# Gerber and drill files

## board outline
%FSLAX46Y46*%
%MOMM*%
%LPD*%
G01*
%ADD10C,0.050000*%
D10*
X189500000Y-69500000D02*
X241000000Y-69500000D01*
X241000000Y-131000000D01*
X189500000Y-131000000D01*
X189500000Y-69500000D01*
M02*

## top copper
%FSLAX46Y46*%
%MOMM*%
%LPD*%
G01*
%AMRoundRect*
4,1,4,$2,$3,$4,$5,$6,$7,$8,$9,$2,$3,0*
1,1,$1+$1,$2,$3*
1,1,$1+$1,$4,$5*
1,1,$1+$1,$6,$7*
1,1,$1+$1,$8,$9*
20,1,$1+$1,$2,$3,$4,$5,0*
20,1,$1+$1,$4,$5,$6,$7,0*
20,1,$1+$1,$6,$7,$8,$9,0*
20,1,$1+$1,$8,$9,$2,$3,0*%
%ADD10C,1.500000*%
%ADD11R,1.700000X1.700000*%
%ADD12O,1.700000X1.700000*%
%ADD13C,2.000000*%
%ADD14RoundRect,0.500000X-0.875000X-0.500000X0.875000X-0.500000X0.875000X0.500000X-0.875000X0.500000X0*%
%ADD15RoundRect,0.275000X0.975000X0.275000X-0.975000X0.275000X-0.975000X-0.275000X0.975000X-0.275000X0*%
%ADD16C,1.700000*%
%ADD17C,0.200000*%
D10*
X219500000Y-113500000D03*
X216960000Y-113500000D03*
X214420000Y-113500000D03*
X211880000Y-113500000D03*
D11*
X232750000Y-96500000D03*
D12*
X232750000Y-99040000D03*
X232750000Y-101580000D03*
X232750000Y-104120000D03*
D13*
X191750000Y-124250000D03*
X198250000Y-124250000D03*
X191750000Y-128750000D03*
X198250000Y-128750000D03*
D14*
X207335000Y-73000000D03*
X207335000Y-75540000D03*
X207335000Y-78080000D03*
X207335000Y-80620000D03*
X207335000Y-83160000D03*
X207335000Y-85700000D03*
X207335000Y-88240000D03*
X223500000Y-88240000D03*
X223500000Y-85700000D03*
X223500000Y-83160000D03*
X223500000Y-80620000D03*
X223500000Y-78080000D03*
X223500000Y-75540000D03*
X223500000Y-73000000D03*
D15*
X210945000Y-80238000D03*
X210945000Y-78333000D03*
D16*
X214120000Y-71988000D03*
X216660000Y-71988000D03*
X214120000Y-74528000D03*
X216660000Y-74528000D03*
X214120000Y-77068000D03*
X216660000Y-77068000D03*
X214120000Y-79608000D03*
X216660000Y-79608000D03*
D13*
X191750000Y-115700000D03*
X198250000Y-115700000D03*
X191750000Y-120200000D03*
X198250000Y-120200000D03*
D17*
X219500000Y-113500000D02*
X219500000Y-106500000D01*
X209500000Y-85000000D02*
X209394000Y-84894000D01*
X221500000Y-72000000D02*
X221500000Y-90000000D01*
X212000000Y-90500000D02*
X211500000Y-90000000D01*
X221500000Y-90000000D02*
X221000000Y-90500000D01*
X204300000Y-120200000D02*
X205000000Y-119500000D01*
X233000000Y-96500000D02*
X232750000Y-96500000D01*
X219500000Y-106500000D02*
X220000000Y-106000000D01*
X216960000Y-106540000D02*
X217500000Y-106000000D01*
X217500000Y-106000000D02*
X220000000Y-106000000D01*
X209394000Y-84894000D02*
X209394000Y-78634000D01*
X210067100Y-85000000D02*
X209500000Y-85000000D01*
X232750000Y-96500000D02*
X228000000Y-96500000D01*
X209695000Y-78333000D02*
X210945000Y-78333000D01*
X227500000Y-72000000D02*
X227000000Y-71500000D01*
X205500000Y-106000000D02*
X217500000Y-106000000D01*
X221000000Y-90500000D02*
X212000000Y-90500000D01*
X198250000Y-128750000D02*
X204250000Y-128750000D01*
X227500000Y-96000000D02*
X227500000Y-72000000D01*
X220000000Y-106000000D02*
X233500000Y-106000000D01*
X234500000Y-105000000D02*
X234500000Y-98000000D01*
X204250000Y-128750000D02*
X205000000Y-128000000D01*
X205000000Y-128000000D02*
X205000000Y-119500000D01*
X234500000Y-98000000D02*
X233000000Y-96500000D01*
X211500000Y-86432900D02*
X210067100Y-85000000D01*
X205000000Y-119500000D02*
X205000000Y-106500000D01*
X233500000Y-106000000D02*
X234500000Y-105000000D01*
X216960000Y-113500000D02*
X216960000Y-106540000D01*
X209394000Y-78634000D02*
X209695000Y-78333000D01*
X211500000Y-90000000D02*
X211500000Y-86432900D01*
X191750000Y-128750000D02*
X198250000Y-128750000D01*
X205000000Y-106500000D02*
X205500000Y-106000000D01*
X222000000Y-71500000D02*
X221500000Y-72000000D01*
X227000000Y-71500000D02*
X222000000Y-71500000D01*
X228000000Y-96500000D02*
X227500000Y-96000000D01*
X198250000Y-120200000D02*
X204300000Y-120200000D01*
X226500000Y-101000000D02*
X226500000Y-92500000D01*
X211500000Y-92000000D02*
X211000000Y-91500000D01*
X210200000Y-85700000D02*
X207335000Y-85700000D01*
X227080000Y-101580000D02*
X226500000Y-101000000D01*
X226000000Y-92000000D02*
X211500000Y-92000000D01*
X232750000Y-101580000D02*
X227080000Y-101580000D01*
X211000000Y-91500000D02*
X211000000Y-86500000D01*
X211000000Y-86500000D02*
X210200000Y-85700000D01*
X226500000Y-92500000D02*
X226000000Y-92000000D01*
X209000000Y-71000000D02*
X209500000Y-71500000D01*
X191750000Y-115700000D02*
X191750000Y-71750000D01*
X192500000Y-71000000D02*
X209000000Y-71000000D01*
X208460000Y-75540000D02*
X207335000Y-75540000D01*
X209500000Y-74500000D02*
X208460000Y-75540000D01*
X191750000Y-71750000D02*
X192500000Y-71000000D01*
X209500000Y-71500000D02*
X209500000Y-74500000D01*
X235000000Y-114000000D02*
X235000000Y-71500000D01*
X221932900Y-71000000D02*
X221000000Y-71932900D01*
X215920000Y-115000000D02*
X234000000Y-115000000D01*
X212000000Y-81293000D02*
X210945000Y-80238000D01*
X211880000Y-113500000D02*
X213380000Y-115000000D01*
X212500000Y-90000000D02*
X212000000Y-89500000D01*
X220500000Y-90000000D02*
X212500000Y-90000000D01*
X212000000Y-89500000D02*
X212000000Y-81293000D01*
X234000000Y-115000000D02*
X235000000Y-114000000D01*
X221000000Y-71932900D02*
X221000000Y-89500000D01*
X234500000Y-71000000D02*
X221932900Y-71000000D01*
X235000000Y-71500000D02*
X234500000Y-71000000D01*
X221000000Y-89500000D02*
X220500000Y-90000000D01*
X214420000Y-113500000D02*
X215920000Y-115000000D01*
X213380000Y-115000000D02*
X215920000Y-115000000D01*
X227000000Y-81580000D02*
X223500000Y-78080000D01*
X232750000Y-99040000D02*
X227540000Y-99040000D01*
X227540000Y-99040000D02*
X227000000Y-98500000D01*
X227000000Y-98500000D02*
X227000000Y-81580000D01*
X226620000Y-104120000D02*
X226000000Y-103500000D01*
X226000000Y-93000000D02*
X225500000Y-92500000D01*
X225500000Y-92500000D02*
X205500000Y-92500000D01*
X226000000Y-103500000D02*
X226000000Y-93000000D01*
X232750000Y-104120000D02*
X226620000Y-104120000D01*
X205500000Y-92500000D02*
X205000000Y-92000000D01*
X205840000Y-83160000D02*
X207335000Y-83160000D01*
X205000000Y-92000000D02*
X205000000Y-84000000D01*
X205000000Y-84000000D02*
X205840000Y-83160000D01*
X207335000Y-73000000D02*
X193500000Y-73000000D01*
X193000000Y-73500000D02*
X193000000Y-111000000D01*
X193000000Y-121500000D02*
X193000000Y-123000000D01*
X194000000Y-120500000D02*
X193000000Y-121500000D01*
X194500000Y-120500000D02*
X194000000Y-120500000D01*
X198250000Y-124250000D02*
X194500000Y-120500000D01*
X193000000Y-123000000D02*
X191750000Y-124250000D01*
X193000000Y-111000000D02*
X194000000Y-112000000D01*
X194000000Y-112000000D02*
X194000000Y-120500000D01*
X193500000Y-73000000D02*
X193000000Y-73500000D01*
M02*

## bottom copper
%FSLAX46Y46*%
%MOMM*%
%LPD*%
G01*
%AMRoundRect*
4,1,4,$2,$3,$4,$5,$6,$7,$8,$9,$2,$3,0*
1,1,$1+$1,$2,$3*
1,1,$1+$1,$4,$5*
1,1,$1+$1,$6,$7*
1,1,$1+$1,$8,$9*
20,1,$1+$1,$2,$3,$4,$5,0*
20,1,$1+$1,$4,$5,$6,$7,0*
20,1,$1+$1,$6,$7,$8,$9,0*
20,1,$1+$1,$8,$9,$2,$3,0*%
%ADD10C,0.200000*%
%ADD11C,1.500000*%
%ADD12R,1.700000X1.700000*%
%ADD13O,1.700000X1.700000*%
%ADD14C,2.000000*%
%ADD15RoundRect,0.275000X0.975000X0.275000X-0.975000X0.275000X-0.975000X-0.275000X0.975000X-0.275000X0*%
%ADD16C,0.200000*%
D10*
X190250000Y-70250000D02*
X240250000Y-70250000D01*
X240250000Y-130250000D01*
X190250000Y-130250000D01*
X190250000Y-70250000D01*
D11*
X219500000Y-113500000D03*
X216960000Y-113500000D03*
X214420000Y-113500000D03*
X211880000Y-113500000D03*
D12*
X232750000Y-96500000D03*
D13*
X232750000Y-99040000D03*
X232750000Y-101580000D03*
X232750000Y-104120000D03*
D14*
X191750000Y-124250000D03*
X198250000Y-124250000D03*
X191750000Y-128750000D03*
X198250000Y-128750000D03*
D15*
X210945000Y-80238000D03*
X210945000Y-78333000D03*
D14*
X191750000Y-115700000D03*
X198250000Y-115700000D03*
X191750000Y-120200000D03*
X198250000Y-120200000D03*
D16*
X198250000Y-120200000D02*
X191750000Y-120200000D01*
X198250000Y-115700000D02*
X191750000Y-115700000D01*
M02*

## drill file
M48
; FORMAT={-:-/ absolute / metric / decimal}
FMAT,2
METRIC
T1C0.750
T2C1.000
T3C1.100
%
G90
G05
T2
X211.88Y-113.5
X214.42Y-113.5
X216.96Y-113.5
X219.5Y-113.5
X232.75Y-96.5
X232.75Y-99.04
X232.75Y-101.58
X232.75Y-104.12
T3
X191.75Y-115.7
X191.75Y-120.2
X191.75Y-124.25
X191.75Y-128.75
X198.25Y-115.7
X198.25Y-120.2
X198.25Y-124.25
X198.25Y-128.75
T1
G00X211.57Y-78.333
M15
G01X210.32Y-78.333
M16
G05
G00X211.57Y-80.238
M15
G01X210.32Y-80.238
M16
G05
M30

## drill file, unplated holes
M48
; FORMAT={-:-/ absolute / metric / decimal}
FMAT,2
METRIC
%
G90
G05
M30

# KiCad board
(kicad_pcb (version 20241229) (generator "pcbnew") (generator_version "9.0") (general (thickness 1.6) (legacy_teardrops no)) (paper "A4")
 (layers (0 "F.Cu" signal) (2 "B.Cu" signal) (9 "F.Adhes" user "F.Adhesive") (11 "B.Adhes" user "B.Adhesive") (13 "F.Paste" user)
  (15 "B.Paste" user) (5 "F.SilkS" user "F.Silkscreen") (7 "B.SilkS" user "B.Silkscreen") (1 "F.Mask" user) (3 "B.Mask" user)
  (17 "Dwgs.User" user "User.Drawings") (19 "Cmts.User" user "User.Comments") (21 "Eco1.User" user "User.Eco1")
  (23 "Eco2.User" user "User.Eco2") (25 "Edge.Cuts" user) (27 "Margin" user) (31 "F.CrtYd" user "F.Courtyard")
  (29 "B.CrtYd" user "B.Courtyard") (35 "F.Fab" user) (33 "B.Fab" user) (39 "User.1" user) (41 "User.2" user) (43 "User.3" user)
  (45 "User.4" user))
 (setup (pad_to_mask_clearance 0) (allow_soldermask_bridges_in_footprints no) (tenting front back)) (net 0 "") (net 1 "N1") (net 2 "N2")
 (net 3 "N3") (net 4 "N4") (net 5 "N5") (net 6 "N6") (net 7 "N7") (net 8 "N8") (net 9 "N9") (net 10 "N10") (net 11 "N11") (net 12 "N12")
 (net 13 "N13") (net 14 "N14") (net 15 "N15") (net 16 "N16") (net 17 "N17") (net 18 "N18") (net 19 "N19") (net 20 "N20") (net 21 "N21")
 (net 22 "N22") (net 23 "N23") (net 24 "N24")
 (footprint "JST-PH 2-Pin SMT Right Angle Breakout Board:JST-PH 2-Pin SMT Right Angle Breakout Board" (layer "F.Cu") (at 206.66 119.59 90)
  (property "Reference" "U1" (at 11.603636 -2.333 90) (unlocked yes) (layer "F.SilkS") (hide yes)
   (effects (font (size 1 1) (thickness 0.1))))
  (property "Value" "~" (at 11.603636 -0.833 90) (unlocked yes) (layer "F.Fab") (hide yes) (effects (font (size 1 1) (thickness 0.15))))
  (pad "1" thru_hole circle (at 6.09 12.84 90) (size 1.5 1.5) (drill 1) (layers "*.Cu" "*.Mask") (remove_unused_layers no) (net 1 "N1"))
  (pad "2" thru_hole circle (at 6.09 10.3 90) (size 1.5 1.5) (drill 1) (layers "*.Cu" "*.Mask") (remove_unused_layers no) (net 1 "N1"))
  (pad "3" thru_hole circle (at 6.09 7.76 90) (size 1.5 1.5) (drill 1) (layers "*.Cu" "*.Mask") (remove_unused_layers no) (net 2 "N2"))
  (pad "4" thru_hole circle (at 6.09 5.22 90) (size 1.5 1.5) (drill 1) (layers "*.Cu" "*.Mask") (remove_unused_layers no) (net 2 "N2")))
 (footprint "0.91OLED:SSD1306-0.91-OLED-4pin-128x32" (layer "F.Cu") (at 196.25 94.31)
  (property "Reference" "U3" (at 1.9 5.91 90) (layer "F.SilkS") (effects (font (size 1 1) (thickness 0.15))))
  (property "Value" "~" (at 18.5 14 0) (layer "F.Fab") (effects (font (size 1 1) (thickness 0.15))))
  (pad "1" thru_hole rect (at 36.5 2.19) (size 1.7 1.7) (drill 1) (layers "*.Cu" "*.Mask") (remove_unused_layers no) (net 1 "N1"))
  (pad "2" thru_hole oval (at 36.5 4.73) (size 1.7 1.7) (drill 1) (layers "*.Cu" "*.Mask") (remove_unused_layers no) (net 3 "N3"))
  (pad "3" thru_hole oval (at 36.5 7.27) (size 1.7 1.7) (drill 1) (layers "*.Cu" "*.Mask") (remove_unused_layers no) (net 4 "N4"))
  (pad "4" thru_hole oval (at 36.5 9.81) (size 1.7 1.7) (drill 1) (layers "*.Cu" "*.Mask") (remove_unused_layers no) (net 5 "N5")))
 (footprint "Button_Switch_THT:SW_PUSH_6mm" (layer "F.Cu") (at 191.75 124.25)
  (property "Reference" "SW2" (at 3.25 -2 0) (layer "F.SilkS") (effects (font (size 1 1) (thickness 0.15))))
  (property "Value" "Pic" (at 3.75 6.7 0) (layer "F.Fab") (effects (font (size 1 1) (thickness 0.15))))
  (pad "1" thru_hole circle (at 0 0 90) (size 2 2) (drill 1.1) (layers "*.Cu" "*.Mask") (remove_unused_layers no) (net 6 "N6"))
  (pad "1" thru_hole circle (at 6.5 0 90) (size 2 2) (drill 1.1) (layers "*.Cu" "*.Mask") (remove_unused_layers no) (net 6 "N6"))
  (pad "2" thru_hole circle (at 0 4.5 90) (size 2 2) (drill 1.1) (layers "*.Cu" "*.Mask") (remove_unused_layers no) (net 1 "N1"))
  (pad "2" thru_hole circle (at 6.5 4.5 90) (size 2 2) (drill 1.1) (layers "*.Cu" "*.Mask") (remove_unused_layers no) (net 1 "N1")))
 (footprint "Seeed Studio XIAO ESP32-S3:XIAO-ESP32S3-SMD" (layer "F.Cu") (at 215.396364 80.573)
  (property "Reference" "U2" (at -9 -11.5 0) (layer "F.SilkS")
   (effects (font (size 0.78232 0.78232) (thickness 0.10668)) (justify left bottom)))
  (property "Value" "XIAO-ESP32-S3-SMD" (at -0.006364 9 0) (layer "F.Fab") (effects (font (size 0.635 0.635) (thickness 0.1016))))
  (pad "1" smd roundrect (at -8.061364 -7.573) (size 2.75 2) (layers "F.Cu" "F.Mask" "F.Paste") (roundrect_rratio 0.25) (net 6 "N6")
   (solder_mask_margin 0.0508) (thermal_bridge_angle 45))
  (pad "2" smd roundrect (at -8.061364 -5.033) (size 2.75 2) (layers "F.Cu" "F.Mask" "F.Paste") (roundrect_rratio 0.25) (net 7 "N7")
   (solder_mask_margin 0.0508) (thermal_bridge_angle 45))
  (pad "3" smd roundrect (at -8.061364 -2.493) (size 2.75 2) (layers "F.Cu" "F.Mask" "F.Paste") (roundrect_rratio 0.25) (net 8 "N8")
   (solder_mask_margin 0.0508) (thermal_bridge_angle 45))
  (pad "4" smd roundrect (at -8.061364 0.047) (size 2.75 2) (layers "F.Cu" "F.Mask" "F.Paste") (roundrect_rratio 0.25) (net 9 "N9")
   (solder_mask_margin 0.0508) (thermal_bridge_angle 45))
  (pad "5" smd roundrect (at -8.061364 2.587) (size 2.75 2) (layers "F.Cu" "F.Mask" "F.Paste") (roundrect_rratio 0.25) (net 5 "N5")
   (solder_mask_margin 0.0508) (thermal_bridge_angle 45))
  (pad "6" smd roundrect (at -8.061364 5.127) (size 2.75 2) (layers "F.Cu" "F.Mask" "F.Paste") (roundrect_rratio 0.25) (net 4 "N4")
   (solder_mask_margin 0.0508) (thermal_bridge_angle 45))
  (pad "7" smd roundrect (at -8.061364 7.667) (size 2.75 2) (layers "F.Cu" "F.Mask" "F.Paste") (roundrect_rratio 0.25) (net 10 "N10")
   (solder_mask_margin 0.0508) (thermal_bridge_angle 45))
  (pad "8" smd roundrect (at 8.103636 7.667) (size 2.75 2) (layers "F.Cu" "F.Mask" "F.Paste") (roundrect_rratio 0.25) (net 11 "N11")
   (solder_mask_margin 0.0508) (thermal_bridge_angle 45))
  (pad "9" smd roundrect (at 8.103636 5.127) (size 2.75 2) (layers "F.Cu" "F.Mask" "F.Paste") (roundrect_rratio 0.25) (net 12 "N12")
   (solder_mask_margin 0.0508) (thermal_bridge_angle 45))
  (pad "10" smd roundrect (at 8.103636 2.587) (size 2.75 2) (layers "F.Cu" "F.Mask" "F.Paste") (roundrect_rratio 0.25) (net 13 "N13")
   (solder_mask_margin 0.0508) (thermal_bridge_angle 45))
  (pad "11" smd roundrect (at 8.103636 0.047) (size 2.75 2) (layers "F.Cu" "F.Mask" "F.Paste") (roundrect_rratio 0.25) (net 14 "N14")
   (solder_mask_margin 0.0508) (thermal_bridge_angle 45))
  (pad "12" smd roundrect (at 8.103636 -2.493) (size 2.75 2) (layers "F.Cu" "F.Mask" "F.Paste") (roundrect_rratio 0.25) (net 3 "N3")
   (solder_mask_margin 0.0508) (thermal_bridge_angle 45))
  (pad "13" smd roundrect (at 8.103636 -5.033) (size 2.75 2) (layers "F.Cu" "F.Mask" "F.Paste") (roundrect_rratio 0.25) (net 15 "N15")
   (solder_mask_margin 0.0508) (thermal_bridge_angle 45))
  (pad "14" smd roundrect (at 8.103636 -7.573) (size 2.75 2) (layers "F.Cu" "F.Mask" "F.Paste") (roundrect_rratio 0.25) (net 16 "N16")
   (solder_mask_margin 0.0508) (thermal_bridge_angle 45))
  (pad "15" thru_hole roundrect (at -4.451364 -0.335 180) (size 2.5 1.1) (drill oval 2 0.75) (layers "*.Cu" "*.Mask")
   (remove_unused_layers no) (roundrect_rratio 0.25) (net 2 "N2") (solder_mask_margin 0.0508) (thermal_bridge_angle 45))
  (pad "16" thru_hole roundrect (at -4.451364 -2.24 180) (size 2.5 1.1) (drill oval 2 0.75) (layers "*.Cu" "*.Mask")
   (remove_unused_layers no) (roundrect_rratio 0.25) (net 1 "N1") (solder_mask_margin 0.0508) (thermal_bridge_angle 45))
  (pad "17" smd circle (at -1.276364 -8.585) (size 1.7 1.7) (layers "F.Cu" "F.Mask" "F.Paste") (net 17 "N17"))
  (pad "18" smd circle (at 1.263636 -8.585) (size 1.7 1.7) (layers "F.Cu" "F.Mask" "F.Paste") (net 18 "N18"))
  (pad "19" smd circle (at -1.276364 -6.045) (size 1.7 1.7) (layers "F.Cu" "F.Mask" "F.Paste") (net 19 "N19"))
  (pad "20" smd circle (at 1.263636 -6.045) (size 1.7 1.7) (layers "F.Cu" "F.Mask" "F.Paste") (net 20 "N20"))
  (pad "21" smd circle (at -1.276364 -3.505) (size 1.7 1.7) (layers "F.Cu" "F.Mask" "F.Paste") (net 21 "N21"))
  (pad "22" smd circle (at 1.263636 -3.505) (size 1.7 1.7) (layers "F.Cu" "F.Mask" "F.Paste") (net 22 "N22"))
  (pad "23" smd circle (at -1.276364 -0.965) (size 1.7 1.7) (layers "F.Cu" "F.Mask" "F.Paste") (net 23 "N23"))
  (pad "24" smd circle (at 1.263636 -0.965) (size 1.7 1.7) (layers "F.Cu" "F.Mask" "F.Paste") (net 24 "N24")))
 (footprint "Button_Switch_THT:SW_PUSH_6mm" (layer "F.Cu") (at 191.75 115.7)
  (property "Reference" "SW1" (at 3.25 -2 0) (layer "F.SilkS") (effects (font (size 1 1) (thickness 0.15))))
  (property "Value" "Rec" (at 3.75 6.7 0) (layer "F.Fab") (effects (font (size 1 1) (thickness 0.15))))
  (pad "1" thru_hole circle (at 0 0 90) (size 2 2) (drill 1.1) (layers "*.Cu" "*.Mask") (remove_unused_layers no) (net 7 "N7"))
  (pad "1" thru_hole circle (at 6.5 0 90) (size 2 2) (drill 1.1) (layers "*.Cu" "*.Mask") (remove_unused_layers no) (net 7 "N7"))
  (pad "2" thru_hole circle (at 0 4.5 90) (size 2 2) (drill 1.1) (layers "*.Cu" "*.Mask") (remove_unused_layers no) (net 1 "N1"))
  (pad "2" thru_hole circle (at 6.5 4.5 90) (size 2 2) (drill 1.1) (layers "*.Cu" "*.Mask") (remove_unused_layers no) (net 1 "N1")))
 (gr_rect (start 190.25 70.25) (end 240.25 130.25) (stroke (width 0.2) (type default)) (fill no) (layer "B.Cu"))
 (gr_rect (start 189.5 69.5) (end 241 131) (stroke (width 0.05) (type default)) (fill no) (layer "Edge.Cuts"))
 (segment (start 219.5 113.5) (end 219.5 106.5) (width 0.2) (layer "F.Cu") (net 1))
 (segment (start 209.5 85) (end 209.394 84.894) (width 0.2) (layer "F.Cu") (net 1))
 (segment (start 221.5 72) (end 221.5 90) (width 0.2) (layer "F.Cu") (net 1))
 (segment (start 212 90.5) (end 211.5 90) (width 0.2) (layer "F.Cu") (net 1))
 (segment (start 221.5 90) (end 221 90.5) (width 0.2) (layer "F.Cu") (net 1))
 (segment (start 204.3 120.2) (end 205 119.5) (width 0.2) (layer "F.Cu") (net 1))
 (segment (start 233 96.5) (end 232.75 96.5) (width 0.2) (layer "F.Cu") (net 1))
 (segment (start 219.5 106.5) (end 220 106) (width 0.2) (layer "F.Cu") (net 1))
 (segment (start 216.96 106.54) (end 217.5 106) (width 0.2) (layer "F.Cu") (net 1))
 (segment (start 217.5 106) (end 220 106) (width 0.2) (layer "F.Cu") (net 1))
 (segment (start 209.394 84.894) (end 209.394 78.634) (width 0.2) (layer "F.Cu") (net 1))
 (segment (start 210.0671 85) (end 209.5 85) (width 0.2) (layer "F.Cu") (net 1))
 (segment (start 232.75 96.5) (end 228 96.5) (width 0.2) (layer "F.Cu") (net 1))
 (segment (start 209.695 78.333) (end 210.945 78.333) (width 0.2) (layer "F.Cu") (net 1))
 (segment (start 227.5 72) (end 227 71.5) (width 0.2) (layer "F.Cu") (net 1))
 (segment (start 205.5 106) (end 217.5 106) (width 0.2) (layer "F.Cu") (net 1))
 (segment (start 221 90.5) (end 212 90.5) (width 0.2) (layer "F.Cu") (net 1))
 (segment (start 198.25 128.75) (end 204.25 128.75) (width 0.2) (layer "F.Cu") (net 1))
 (segment (start 227.5 96) (end 227.5 72) (width 0.2) (layer "F.Cu") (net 1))
 (segment (start 220 106) (end 233.5 106) (width 0.2) (layer "F.Cu") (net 1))
 (segment (start 234.5 105) (end 234.5 98) (width 0.2) (layer "F.Cu") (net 1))
 (segment (start 204.25 128.75) (end 205 128) (width 0.2) (layer "F.Cu") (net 1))
 (segment (start 205 128) (end 205 119.5) (width 0.2) (layer "F.Cu") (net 1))
 (segment (start 234.5 98) (end 233 96.5) (width 0.2) (layer "F.Cu") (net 1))
 (segment (start 211.5 86.4329) (end 210.0671 85) (width 0.2) (layer "F.Cu") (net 1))
 (segment (start 205 119.5) (end 205 106.5) (width 0.2) (layer "F.Cu") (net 1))
 (segment (start 233.5 106) (end 234.5 105) (width 0.2) (layer "F.Cu") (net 1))
 (segment (start 216.96 113.5) (end 216.96 106.54) (width 0.2) (layer "F.Cu") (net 1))
 (segment (start 209.394 78.634) (end 209.695 78.333) (width 0.2) (layer "F.Cu") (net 1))
 (segment (start 211.5 90) (end 211.5 86.4329) (width 0.2) (layer "F.Cu") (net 1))
 (segment (start 191.75 128.75) (end 198.25 128.75) (width 0.2) (layer "F.Cu") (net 1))
 (segment (start 205 106.5) (end 205.5 106) (width 0.2) (layer "F.Cu") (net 1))
 (segment (start 222 71.5) (end 221.5 72) (width 0.2) (layer "F.Cu") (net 1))
 (segment (start 227 71.5) (end 222 71.5) (width 0.2) (layer "F.Cu") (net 1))
 (segment (start 228 96.5) (end 227.5 96) (width 0.2) (layer "F.Cu") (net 1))
 (segment (start 198.25 120.2) (end 204.3 120.2) (width 0.2) (layer "F.Cu") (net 1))
 (segment (start 198.25 120.2) (end 191.75 120.2) (width 0.2) (layer "B.Cu") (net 1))
 (segment (start 226.5 101) (end 226.5 92.5) (width 0.2) (layer "F.Cu") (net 4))
 (segment (start 211.5 92) (end 211 91.5) (width 0.2) (layer "F.Cu") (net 4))
 (segment (start 210.2 85.7) (end 207.335 85.7) (width 0.2) (layer "F.Cu") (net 4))
 (segment (start 227.08 101.58) (end 226.5 101) (width 0.2) (layer "F.Cu") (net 4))
 (segment (start 226 92) (end 211.5 92) (width 0.2) (layer "F.Cu") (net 4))
 (segment (start 232.75 101.58) (end 227.08 101.58) (width 0.2) (layer "F.Cu") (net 4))
 (segment (start 211 91.5) (end 211 86.5) (width 0.2) (layer "F.Cu") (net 4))
 (segment (start 211 86.5) (end 210.2 85.7) (width 0.2) (layer "F.Cu") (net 4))
 (segment (start 226.5 92.5) (end 226 92) (width 0.2) (layer "F.Cu") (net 4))
 (segment (start 209 71) (end 209.5 71.5) (width 0.2) (layer "F.Cu") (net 7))
 (segment (start 191.75 115.7) (end 191.75 71.75) (width 0.2) (layer "F.Cu") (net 7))
 (segment (start 192.5 71) (end 209 71) (width 0.2) (layer "F.Cu") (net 7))
 (segment (start 208.46 75.54) (end 207.335 75.54) (width 0.2) (layer "F.Cu") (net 7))
 (segment (start 209.5 74.5) (end 208.46 75.54) (width 0.2) (layer "F.Cu") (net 7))
 (segment (start 191.75 71.75) (end 192.5 71) (width 0.2) (layer "F.Cu") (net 7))
 (segment (start 209.5 71.5) (end 209.5 74.5) (width 0.2) (layer "F.Cu") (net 7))
 (segment (start 198.25 115.7) (end 191.75 115.7) (width 0.2) (layer "B.Cu") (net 7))
 (segment (start 235 114) (end 235 71.5) (width 0.2) (layer "F.Cu") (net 2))
 (segment (start 221.9329 71) (end 221 71.9329) (width 0.2) (layer "F.Cu") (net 2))
 (segment (start 215.92 115) (end 234 115) (width 0.2) (layer "F.Cu") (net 2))
 (segment (start 212 81.293) (end 210.945 80.238) (width 0.2) (layer "F.Cu") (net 2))
 (segment (start 211.88 113.5) (end 213.38 115) (width 0.2) (layer "F.Cu") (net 2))
 (segment (start 212.5 90) (end 212 89.5) (width 0.2) (layer "F.Cu") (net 2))
 (segment (start 220.5 90) (end 212.5 90) (width 0.2) (layer "F.Cu") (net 2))
 (segment (start 212 89.5) (end 212 81.293) (width 0.2) (layer "F.Cu") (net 2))
 (segment (start 234 115) (end 235 114) (width 0.2) (layer "F.Cu") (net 2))
 (segment (start 221 71.9329) (end 221 89.5) (width 0.2) (layer "F.Cu") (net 2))
 (segment (start 234.5 71) (end 221.9329 71) (width 0.2) (layer "F.Cu") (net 2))
 (segment (start 235 71.5) (end 234.5 71) (width 0.2) (layer "F.Cu") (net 2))
 (segment (start 221 89.5) (end 220.5 90) (width 0.2) (layer "F.Cu") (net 2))
 (segment (start 214.42 113.5) (end 215.92 115) (width 0.2) (layer "F.Cu") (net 2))
 (segment (start 213.38 115) (end 215.92 115) (width 0.2) (layer "F.Cu") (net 2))
 (segment (start 227 81.58) (end 223.5 78.08) (width 0.2) (layer "F.Cu") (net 3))
 (segment (start 232.75 99.04) (end 227.54 99.04) (width 0.2) (layer "F.Cu") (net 3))
 (segment (start 227.54 99.04) (end 227 98.5) (width 0.2) (layer "F.Cu") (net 3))
 (segment (start 227 98.5) (end 227 81.58) (width 0.2) (layer "F.Cu") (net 3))
 (segment (start 226.62 104.12) (end 226 103.5) (width 0.2) (layer "F.Cu") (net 5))
 (segment (start 226 93) (end 225.5 92.5) (width 0.2) (layer "F.Cu") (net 5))
 (segment (start 225.5 92.5) (end 205.5 92.5) (width 0.2) (layer "F.Cu") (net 5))
 (segment (start 226 103.5) (end 226 93) (width 0.2) (layer "F.Cu") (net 5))
 (segment (start 232.75 104.12) (end 226.62 104.12) (width 0.2) (layer "F.Cu") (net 5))
 (segment (start 205.5 92.5) (end 205 92) (width 0.2) (layer "F.Cu") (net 5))
 (segment (start 205.84 83.16) (end 207.335 83.16) (width 0.2) (layer "F.Cu") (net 5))
 (segment (start 205 92) (end 205 84) (width 0.2) (layer "F.Cu") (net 5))
 (segment (start 205 84) (end 205.84 83.16) (width 0.2) (layer "F.Cu") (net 5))
 (segment (start 207.335 73) (end 193.5 73) (width 0.2) (layer "F.Cu") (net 6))
 (segment (start 193 73.5) (end 193 111) (width 0.2) (layer "F.Cu") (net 6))
 (segment (start 193 121.5) (end 193 123) (width 0.2) (layer "F.Cu") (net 6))
 (segment (start 194 120.5) (end 193 121.5) (width 0.2) (layer "F.Cu") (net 6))
 (segment (start 194.5 120.5) (end 194 120.5) (width 0.2) (layer "F.Cu") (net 6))
 (segment (start 198.25 124.25) (end 194.5 120.5) (width 0.2) (layer "F.Cu") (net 6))
 (segment (start 193 123) (end 191.75 124.25) (width 0.2) (layer "F.Cu") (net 6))
 (segment (start 193 111) (end 194 112) (width 0.2) (layer "F.Cu") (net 6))
 (segment (start 194 112) (end 194 120.5) (width 0.2) (layer "F.Cu") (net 6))
 (segment (start 193.5 73) (end 193 73.5) (width 0.2) (layer "F.Cu") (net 6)))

